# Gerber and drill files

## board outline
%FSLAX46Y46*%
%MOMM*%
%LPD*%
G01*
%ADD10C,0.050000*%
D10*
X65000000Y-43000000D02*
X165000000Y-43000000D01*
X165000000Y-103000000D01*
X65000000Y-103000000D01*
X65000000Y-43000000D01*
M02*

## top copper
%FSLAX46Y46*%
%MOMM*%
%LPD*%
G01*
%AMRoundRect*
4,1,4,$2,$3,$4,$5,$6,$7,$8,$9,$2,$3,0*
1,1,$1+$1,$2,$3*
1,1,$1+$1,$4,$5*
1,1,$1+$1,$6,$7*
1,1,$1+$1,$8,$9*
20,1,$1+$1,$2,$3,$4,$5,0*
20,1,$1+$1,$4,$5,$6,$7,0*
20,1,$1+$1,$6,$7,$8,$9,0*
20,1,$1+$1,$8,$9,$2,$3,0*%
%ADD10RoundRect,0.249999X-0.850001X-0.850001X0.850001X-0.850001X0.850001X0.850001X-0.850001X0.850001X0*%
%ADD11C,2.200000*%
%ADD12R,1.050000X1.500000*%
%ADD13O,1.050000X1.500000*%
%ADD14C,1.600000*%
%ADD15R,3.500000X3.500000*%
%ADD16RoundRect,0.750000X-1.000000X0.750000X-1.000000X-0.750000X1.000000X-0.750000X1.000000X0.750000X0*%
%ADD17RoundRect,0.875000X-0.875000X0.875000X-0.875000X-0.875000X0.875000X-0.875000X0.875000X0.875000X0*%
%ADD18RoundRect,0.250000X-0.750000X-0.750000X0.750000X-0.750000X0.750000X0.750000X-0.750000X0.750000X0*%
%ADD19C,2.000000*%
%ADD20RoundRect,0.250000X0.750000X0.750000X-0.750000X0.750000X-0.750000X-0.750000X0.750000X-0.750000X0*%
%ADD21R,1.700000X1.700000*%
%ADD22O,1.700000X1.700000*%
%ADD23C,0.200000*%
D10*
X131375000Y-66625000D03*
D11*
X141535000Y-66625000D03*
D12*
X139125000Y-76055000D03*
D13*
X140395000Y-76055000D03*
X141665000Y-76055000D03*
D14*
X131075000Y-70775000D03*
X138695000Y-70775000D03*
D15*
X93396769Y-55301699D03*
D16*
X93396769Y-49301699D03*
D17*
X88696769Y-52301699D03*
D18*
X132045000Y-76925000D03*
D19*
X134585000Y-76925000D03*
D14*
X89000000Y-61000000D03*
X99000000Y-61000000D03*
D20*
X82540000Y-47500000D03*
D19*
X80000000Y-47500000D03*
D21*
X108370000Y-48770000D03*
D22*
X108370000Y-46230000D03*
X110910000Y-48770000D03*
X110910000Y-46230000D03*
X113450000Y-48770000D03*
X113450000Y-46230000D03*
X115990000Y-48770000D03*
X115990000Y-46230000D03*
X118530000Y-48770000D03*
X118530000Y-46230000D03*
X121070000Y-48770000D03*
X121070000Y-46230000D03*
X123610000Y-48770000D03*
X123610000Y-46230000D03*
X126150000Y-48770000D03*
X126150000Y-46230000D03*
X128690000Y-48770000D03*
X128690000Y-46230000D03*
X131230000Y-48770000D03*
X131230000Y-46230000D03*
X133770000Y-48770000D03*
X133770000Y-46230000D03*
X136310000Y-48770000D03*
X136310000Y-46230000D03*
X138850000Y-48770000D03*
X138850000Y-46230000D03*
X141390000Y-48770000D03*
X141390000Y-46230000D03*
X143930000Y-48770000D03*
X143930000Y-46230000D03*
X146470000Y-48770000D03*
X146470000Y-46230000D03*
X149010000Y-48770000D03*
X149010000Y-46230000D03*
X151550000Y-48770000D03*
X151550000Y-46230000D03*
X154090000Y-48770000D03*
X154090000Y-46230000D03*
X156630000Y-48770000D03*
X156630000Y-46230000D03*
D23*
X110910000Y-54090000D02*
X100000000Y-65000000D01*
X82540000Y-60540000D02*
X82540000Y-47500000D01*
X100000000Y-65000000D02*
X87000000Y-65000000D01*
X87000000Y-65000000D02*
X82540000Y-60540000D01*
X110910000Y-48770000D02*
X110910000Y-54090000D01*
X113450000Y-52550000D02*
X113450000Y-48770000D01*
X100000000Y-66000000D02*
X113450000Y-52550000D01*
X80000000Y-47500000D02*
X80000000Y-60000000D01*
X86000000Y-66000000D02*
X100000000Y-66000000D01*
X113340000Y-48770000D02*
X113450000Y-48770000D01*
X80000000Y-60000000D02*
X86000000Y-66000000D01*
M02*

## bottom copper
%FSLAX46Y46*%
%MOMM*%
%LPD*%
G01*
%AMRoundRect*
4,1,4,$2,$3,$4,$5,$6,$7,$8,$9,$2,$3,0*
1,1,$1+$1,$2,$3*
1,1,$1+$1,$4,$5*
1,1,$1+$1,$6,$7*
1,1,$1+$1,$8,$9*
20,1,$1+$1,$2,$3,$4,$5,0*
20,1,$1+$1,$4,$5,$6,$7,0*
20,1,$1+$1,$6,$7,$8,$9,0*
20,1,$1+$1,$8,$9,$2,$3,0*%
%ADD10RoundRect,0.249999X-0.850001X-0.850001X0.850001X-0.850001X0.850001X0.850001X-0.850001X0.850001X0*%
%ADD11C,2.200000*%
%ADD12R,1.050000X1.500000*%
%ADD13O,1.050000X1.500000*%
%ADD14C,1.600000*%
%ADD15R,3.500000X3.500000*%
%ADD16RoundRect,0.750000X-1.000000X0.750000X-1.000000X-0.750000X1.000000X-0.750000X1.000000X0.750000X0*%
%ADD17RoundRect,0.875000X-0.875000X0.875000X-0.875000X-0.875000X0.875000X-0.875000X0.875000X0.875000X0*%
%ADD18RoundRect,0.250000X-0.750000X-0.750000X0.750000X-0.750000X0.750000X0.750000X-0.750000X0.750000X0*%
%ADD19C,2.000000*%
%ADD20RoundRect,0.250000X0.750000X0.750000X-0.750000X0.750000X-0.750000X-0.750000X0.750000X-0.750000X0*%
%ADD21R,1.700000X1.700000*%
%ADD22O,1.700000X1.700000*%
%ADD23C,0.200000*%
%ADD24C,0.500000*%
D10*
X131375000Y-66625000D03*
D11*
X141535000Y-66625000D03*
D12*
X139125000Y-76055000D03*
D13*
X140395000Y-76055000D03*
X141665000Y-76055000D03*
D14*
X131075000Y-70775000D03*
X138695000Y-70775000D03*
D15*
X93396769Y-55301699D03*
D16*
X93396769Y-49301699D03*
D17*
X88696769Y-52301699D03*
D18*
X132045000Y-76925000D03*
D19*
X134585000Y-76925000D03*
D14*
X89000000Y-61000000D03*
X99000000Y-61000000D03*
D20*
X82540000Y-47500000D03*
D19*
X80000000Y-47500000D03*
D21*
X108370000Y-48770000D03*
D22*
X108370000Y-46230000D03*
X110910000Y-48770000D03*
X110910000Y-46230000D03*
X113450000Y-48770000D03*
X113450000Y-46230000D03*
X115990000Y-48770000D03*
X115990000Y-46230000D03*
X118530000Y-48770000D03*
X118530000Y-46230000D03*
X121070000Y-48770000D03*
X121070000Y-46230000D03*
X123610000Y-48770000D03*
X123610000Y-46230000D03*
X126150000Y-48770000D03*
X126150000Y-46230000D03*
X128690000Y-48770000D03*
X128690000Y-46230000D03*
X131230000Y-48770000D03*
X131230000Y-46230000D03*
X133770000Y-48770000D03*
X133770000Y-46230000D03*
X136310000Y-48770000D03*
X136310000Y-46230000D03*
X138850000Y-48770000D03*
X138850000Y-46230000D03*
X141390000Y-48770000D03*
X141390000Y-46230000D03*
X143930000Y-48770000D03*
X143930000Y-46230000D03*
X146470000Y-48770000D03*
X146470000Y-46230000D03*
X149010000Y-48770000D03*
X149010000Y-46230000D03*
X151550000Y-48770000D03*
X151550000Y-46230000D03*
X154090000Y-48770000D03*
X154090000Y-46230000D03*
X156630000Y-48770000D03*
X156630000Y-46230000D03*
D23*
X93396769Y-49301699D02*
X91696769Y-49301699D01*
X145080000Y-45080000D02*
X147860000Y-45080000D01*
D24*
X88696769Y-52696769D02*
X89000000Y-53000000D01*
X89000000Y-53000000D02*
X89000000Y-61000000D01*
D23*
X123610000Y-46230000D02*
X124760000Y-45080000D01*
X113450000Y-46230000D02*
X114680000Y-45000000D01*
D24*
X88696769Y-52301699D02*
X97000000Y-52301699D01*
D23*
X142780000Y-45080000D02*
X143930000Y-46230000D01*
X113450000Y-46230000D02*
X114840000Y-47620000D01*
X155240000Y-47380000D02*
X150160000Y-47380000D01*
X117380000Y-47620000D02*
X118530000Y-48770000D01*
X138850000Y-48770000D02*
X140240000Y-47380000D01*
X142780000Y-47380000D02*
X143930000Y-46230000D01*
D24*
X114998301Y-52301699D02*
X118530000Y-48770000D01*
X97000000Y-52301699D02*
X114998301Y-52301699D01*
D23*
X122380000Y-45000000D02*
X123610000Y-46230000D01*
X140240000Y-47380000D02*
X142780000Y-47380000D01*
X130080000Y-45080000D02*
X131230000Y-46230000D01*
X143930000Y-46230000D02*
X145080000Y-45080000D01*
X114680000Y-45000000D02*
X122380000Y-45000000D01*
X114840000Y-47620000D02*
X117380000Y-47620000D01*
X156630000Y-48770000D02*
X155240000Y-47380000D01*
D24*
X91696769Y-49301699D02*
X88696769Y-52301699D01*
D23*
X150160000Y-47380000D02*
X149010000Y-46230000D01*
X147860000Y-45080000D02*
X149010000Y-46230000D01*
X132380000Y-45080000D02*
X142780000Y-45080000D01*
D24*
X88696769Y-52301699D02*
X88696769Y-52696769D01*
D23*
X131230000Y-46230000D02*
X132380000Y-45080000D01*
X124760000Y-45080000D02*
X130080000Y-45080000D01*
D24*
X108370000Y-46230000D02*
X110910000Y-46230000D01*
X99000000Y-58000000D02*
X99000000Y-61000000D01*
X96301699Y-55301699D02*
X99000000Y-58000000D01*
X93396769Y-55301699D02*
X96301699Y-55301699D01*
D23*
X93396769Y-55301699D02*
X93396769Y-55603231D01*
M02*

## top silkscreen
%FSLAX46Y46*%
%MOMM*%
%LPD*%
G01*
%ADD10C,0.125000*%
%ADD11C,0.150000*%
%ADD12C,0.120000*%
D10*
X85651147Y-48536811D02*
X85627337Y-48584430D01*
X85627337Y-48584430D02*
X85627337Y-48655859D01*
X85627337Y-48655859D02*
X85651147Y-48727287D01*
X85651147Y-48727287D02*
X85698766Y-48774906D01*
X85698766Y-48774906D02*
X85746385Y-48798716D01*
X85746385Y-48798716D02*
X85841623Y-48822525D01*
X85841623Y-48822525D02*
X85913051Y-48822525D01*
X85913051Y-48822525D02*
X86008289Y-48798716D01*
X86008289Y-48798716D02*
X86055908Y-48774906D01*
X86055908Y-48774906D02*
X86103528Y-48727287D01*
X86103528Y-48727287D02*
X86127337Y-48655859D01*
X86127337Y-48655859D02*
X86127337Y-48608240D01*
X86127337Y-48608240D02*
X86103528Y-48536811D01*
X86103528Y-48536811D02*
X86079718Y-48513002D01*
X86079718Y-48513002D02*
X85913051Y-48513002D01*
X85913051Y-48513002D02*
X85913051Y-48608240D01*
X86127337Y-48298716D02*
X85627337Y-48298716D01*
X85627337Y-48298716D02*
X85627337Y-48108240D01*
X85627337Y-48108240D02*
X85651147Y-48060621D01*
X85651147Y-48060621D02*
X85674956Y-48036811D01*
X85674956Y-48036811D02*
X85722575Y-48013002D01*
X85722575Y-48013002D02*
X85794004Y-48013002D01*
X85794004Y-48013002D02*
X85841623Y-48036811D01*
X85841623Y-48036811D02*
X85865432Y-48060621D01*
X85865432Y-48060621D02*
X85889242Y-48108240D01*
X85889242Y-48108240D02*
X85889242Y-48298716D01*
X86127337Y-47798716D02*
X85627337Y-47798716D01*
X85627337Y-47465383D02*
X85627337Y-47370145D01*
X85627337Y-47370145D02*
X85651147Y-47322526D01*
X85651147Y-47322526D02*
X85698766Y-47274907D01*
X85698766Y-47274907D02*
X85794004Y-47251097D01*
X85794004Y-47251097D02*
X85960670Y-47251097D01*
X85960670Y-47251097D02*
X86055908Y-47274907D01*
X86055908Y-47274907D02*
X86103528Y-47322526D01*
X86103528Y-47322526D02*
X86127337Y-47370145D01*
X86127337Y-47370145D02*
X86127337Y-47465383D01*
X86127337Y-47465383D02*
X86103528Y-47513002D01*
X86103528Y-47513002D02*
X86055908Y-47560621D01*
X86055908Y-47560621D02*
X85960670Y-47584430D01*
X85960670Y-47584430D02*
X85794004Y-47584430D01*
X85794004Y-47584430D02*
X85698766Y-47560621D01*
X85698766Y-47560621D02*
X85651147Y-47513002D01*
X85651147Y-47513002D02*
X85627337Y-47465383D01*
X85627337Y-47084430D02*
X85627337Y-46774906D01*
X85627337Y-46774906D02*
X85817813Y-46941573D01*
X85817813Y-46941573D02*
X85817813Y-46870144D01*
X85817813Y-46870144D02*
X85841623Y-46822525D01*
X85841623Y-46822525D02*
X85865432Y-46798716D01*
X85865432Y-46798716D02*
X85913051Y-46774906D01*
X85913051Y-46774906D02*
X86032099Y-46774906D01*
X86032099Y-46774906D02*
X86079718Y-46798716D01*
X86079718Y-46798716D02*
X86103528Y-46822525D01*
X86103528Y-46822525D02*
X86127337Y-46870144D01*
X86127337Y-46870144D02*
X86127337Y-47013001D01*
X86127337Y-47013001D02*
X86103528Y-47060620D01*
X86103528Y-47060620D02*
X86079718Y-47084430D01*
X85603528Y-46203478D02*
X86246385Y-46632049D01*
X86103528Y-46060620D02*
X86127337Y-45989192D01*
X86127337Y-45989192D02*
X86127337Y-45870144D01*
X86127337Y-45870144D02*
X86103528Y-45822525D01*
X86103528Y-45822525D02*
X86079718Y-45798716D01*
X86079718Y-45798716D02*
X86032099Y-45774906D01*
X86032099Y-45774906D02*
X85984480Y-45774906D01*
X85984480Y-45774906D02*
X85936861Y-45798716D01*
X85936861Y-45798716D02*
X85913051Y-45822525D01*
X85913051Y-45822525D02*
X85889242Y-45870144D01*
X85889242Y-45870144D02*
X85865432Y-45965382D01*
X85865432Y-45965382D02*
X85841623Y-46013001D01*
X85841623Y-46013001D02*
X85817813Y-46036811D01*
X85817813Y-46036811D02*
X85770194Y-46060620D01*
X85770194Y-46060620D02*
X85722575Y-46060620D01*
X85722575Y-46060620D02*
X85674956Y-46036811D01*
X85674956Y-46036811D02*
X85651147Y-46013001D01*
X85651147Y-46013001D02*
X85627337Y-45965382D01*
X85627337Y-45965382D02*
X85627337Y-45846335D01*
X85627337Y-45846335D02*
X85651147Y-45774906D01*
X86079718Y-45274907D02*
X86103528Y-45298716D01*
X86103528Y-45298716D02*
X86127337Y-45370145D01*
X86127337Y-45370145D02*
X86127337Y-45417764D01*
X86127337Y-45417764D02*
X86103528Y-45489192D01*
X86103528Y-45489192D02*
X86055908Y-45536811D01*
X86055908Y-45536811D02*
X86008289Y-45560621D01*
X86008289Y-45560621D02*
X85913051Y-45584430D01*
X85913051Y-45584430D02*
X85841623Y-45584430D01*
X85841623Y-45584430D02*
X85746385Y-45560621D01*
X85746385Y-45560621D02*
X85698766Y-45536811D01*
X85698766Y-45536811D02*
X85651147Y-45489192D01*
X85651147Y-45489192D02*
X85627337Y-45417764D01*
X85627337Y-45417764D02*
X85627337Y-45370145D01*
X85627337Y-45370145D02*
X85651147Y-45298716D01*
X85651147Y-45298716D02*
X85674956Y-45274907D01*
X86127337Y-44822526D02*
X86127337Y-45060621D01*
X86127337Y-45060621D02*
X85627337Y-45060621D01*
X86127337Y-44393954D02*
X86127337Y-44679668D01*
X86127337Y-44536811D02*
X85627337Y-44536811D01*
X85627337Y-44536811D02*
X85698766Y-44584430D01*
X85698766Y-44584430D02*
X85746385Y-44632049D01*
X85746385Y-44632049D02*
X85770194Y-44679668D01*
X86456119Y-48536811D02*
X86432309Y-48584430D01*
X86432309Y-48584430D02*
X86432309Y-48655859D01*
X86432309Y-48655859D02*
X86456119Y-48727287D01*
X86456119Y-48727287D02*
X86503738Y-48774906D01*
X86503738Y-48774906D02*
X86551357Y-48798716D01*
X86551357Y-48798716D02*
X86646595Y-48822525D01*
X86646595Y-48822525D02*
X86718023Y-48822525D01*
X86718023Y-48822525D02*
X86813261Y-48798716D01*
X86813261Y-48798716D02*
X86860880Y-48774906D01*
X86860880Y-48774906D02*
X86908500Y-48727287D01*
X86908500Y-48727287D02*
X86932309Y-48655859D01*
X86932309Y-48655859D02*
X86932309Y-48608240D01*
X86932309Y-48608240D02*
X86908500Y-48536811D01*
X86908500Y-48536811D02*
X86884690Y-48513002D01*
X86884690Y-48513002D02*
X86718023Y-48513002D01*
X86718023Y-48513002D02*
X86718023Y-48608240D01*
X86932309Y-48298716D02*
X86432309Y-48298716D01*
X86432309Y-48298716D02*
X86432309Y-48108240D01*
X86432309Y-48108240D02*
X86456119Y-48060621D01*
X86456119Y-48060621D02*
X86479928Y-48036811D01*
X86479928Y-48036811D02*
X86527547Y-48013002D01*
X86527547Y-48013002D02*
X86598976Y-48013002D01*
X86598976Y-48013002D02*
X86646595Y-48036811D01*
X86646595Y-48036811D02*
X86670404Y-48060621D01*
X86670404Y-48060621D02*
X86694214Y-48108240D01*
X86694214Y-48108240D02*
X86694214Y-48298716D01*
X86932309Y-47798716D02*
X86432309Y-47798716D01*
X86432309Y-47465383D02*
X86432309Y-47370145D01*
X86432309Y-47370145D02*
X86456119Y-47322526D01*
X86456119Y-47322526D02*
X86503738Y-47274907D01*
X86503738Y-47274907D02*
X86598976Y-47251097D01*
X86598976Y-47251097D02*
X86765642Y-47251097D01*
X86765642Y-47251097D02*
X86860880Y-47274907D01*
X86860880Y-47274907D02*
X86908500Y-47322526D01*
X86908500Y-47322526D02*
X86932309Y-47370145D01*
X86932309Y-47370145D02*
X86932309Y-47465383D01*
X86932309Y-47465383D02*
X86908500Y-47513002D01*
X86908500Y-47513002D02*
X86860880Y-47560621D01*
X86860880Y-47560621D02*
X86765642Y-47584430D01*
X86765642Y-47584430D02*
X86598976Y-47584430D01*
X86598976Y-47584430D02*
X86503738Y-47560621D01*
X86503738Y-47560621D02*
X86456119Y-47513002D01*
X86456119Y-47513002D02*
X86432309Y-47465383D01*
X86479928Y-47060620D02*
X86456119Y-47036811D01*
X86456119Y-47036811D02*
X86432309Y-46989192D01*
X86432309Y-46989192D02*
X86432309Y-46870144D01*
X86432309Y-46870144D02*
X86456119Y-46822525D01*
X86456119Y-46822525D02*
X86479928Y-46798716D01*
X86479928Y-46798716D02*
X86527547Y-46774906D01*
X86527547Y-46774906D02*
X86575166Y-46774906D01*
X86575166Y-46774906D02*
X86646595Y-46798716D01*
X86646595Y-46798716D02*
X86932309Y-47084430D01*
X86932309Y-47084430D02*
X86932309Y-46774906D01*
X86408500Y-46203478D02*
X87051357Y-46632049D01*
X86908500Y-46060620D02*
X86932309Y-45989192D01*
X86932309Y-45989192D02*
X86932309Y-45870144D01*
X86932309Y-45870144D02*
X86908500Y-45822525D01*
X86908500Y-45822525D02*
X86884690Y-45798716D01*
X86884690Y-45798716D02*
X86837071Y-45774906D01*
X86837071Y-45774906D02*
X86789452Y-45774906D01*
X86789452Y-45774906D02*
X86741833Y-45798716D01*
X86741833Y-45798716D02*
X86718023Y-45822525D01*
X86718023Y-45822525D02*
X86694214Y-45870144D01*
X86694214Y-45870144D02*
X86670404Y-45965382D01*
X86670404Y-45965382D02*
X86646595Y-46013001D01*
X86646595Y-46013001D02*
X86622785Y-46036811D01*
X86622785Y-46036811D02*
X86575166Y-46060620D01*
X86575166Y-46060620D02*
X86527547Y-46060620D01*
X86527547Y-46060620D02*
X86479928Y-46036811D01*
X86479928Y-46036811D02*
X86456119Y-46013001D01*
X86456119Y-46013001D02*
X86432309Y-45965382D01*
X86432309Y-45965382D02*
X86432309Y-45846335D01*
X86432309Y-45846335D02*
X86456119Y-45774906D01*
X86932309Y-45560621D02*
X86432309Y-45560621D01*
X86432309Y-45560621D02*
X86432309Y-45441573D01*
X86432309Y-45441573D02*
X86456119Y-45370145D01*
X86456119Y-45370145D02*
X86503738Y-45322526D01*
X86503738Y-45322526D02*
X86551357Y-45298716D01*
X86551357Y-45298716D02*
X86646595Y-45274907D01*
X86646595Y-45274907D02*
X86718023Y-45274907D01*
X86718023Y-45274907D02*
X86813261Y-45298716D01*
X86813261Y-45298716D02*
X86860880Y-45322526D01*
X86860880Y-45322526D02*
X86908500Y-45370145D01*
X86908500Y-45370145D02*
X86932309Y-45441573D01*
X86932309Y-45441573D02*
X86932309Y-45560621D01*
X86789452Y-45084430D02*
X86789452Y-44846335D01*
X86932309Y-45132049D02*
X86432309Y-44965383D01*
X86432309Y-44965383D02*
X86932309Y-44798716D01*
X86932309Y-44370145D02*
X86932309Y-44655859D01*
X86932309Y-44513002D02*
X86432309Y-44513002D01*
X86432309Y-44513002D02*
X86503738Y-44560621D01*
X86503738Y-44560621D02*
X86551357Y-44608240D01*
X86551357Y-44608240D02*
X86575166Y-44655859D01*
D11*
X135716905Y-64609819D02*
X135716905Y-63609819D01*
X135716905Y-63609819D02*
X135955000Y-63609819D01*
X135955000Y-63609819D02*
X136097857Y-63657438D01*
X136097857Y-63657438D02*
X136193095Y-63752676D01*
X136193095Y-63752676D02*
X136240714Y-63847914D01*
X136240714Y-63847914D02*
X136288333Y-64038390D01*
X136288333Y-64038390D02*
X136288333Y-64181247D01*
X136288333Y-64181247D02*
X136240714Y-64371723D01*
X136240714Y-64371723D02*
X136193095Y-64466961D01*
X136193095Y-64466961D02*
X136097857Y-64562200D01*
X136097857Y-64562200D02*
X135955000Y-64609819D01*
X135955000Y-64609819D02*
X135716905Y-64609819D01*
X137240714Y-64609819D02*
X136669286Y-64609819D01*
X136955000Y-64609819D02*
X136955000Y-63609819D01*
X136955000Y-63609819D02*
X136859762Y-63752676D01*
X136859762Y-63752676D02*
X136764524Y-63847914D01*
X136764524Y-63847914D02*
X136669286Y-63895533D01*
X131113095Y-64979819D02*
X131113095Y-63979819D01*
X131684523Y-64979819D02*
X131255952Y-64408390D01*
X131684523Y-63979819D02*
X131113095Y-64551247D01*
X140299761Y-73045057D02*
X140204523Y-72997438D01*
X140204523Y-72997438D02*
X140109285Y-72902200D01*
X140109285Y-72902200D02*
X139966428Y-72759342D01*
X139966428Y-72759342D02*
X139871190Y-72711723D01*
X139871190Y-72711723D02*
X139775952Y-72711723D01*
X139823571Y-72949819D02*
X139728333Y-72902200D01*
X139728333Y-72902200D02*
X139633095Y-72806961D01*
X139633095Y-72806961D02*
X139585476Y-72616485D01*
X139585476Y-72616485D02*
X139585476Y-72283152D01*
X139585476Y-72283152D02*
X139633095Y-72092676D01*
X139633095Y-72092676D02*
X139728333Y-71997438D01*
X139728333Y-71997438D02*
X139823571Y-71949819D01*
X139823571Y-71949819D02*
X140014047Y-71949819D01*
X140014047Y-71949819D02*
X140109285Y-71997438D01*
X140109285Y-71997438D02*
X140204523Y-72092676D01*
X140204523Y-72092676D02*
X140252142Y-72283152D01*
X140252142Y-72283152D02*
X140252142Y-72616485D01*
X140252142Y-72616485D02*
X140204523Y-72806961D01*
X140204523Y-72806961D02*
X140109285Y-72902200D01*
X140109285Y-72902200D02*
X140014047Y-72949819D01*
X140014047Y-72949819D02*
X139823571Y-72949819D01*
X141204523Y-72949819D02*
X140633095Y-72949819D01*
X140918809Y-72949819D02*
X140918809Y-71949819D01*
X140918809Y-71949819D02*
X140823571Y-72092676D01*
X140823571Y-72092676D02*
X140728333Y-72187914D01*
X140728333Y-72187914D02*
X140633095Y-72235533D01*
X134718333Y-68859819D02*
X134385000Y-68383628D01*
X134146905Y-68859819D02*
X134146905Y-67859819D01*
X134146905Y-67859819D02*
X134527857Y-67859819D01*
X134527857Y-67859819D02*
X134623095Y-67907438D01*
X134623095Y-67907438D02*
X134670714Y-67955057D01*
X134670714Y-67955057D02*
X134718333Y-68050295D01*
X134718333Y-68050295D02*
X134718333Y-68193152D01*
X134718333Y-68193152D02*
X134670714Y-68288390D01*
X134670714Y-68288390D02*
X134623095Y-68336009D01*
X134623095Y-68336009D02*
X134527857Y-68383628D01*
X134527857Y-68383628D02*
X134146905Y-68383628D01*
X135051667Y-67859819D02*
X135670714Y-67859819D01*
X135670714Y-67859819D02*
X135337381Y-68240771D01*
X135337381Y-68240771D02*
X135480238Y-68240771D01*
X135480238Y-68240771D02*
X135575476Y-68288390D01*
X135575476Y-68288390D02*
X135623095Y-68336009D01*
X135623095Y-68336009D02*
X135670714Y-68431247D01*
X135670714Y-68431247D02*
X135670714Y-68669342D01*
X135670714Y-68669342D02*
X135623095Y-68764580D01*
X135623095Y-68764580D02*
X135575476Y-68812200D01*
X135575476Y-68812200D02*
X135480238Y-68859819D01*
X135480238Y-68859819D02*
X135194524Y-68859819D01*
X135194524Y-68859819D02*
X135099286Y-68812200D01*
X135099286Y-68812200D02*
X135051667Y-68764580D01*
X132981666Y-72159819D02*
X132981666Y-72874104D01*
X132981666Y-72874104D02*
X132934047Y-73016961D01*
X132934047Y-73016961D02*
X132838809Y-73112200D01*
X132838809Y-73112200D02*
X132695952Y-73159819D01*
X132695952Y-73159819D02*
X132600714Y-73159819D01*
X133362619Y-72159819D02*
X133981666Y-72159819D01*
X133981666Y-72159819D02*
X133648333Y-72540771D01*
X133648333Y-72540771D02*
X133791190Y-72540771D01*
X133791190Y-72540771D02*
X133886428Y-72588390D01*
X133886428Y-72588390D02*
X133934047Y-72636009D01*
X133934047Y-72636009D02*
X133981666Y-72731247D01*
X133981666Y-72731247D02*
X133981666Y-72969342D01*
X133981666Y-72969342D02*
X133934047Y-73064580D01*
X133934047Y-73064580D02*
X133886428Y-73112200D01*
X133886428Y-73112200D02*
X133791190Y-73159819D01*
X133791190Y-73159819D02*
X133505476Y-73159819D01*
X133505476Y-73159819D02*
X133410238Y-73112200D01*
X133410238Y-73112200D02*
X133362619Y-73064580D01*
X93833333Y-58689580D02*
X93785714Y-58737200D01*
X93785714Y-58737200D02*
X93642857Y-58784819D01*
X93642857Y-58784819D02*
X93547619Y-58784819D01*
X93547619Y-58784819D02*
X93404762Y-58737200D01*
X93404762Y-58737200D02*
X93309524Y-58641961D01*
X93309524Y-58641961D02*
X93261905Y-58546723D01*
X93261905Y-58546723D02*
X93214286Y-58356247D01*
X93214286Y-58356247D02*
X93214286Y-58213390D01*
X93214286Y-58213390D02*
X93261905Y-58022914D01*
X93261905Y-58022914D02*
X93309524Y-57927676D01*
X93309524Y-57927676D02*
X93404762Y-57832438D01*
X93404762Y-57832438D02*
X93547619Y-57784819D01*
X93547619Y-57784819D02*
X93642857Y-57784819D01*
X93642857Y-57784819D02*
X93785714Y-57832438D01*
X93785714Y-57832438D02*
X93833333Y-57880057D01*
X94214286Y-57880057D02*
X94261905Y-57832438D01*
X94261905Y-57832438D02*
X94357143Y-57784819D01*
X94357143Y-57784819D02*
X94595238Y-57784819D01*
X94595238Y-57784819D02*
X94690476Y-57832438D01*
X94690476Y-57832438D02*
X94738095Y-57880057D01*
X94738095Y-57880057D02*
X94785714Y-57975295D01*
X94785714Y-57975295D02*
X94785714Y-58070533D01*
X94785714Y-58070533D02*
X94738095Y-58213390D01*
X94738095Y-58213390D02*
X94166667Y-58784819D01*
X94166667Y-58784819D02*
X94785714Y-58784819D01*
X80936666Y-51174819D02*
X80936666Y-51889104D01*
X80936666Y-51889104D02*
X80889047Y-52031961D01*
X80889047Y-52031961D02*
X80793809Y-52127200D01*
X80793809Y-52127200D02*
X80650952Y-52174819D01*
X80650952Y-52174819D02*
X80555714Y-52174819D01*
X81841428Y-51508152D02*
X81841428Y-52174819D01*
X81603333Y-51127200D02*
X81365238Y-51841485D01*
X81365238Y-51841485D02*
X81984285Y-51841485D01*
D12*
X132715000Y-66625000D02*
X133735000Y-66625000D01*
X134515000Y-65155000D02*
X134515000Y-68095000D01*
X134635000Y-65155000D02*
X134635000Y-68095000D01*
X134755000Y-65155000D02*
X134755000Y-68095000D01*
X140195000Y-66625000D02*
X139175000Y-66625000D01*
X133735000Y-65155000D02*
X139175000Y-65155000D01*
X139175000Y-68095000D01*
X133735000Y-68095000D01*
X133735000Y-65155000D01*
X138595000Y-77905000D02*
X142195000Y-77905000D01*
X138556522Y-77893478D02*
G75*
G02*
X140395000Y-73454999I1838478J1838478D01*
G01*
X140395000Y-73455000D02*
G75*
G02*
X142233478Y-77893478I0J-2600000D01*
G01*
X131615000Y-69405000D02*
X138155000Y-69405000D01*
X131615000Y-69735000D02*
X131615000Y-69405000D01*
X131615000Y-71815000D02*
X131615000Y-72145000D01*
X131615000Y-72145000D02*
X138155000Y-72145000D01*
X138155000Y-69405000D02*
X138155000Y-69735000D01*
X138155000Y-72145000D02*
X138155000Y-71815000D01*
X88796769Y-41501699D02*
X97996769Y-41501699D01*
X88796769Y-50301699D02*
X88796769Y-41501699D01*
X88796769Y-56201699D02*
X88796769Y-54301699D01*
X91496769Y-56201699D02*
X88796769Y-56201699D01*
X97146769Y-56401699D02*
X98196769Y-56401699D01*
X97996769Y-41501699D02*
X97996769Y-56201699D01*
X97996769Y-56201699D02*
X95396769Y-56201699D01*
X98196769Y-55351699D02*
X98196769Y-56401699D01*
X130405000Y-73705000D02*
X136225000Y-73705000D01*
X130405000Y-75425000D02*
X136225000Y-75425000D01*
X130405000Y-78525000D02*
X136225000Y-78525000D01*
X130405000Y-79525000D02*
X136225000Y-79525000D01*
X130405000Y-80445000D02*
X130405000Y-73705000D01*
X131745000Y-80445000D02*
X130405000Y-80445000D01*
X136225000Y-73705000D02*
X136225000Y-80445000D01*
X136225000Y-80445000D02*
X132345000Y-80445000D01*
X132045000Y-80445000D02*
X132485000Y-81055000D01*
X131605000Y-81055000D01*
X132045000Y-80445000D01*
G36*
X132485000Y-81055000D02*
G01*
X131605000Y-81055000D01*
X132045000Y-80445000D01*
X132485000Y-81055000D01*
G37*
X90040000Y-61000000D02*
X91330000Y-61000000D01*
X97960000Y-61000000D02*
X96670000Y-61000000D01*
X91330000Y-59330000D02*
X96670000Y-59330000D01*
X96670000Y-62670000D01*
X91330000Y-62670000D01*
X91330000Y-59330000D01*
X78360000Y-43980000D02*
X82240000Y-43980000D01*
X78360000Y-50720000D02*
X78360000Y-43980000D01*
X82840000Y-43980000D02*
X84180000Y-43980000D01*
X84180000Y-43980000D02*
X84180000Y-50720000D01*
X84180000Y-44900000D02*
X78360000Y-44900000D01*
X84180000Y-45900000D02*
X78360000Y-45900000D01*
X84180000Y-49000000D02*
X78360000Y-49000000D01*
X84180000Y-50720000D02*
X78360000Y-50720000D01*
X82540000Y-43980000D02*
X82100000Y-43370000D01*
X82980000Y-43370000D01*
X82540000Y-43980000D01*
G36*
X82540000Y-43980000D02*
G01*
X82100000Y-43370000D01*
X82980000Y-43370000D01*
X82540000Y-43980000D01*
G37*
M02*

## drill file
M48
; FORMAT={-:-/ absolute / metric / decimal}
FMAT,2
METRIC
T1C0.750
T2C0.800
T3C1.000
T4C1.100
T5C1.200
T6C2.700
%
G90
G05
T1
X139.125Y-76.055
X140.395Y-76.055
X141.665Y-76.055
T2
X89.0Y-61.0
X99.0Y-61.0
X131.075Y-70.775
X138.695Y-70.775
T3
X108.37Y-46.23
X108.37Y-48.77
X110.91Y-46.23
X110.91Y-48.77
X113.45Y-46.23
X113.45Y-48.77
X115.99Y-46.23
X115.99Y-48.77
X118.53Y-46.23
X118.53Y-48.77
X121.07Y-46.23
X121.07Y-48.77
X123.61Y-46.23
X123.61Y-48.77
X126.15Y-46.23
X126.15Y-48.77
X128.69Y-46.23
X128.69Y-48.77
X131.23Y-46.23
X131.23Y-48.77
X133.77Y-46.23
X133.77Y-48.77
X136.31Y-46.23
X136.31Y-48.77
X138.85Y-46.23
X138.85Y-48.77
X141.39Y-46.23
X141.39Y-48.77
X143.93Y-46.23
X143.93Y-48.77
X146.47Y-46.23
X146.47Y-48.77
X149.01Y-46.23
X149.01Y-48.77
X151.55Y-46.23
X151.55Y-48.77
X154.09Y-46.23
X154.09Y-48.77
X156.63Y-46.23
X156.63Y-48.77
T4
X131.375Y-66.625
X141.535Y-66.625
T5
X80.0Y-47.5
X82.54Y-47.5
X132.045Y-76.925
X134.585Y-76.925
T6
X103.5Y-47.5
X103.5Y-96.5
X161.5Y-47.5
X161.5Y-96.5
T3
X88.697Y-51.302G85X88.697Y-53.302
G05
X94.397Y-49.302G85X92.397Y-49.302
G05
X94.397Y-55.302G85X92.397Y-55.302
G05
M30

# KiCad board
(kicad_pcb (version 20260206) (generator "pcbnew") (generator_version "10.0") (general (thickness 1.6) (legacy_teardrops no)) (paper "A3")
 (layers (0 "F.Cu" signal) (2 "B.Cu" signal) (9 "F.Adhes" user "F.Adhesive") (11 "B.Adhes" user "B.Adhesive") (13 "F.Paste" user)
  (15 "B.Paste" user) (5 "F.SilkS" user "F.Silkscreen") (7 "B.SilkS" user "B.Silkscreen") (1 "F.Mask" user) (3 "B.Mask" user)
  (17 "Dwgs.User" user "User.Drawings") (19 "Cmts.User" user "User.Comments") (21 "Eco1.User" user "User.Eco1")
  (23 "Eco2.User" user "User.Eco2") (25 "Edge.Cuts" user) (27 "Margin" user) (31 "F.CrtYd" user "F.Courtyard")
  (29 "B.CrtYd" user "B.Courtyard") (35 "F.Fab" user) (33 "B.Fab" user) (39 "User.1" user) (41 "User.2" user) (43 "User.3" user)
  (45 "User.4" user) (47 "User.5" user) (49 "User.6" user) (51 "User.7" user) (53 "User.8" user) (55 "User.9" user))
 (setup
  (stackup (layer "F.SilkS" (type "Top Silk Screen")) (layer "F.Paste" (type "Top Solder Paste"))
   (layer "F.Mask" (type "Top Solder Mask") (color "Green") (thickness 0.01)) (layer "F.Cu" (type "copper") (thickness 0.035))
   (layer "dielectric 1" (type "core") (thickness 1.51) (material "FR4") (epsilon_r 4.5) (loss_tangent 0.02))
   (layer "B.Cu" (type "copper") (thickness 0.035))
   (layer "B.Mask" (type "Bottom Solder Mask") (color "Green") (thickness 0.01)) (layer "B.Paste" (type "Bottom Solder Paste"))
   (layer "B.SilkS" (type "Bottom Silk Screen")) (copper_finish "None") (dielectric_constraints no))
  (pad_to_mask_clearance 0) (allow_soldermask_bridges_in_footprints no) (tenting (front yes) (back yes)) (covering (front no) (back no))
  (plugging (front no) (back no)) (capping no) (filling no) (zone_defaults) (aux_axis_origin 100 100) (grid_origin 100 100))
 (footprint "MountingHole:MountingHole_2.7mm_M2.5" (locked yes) (layer "F.Cu") (at 161.5 47.5)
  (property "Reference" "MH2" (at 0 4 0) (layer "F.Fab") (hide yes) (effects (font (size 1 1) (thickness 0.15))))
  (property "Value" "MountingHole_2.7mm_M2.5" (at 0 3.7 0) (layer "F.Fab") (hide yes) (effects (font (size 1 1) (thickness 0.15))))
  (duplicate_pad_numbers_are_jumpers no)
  (pad "" np_thru_hole circle (at 0 0) (size 2.7 2.7) (drill 2.7) (layers "*.Cu" "*.Mask")))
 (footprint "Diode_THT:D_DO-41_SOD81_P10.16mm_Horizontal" (layer "F.Cu") (at 131.375 66.625)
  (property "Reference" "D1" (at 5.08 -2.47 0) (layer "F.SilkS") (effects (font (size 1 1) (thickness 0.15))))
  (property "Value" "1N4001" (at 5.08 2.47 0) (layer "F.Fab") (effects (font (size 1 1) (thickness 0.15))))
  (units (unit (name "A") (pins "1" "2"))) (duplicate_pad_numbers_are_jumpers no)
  (fp_line (start 1.34 0) (end 2.36 0) (stroke (width 0.12) (type solid)) (layer "F.SilkS"))
  (fp_line (start 3.14 -1.47) (end 3.14 1.47) (stroke (width 0.12) (type solid)) (layer "F.SilkS"))
  (fp_line (start 3.26 -1.47) (end 3.26 1.47) (stroke (width 0.12) (type solid)) (layer "F.SilkS"))
  (fp_line (start 3.38 -1.47) (end 3.38 1.47) (stroke (width 0.12) (type solid)) (layer "F.SilkS"))
  (fp_line (start 8.82 0) (end 7.8 0) (stroke (width 0.12) (type solid)) (layer "F.SilkS"))
  (fp_rect (start 2.36 -1.47) (end 7.8 1.47) (stroke (width 0.12) (type solid)) (fill no) (layer "F.SilkS"))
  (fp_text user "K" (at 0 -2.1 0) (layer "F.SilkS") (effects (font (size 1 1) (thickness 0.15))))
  (pad "1" thru_hole roundrect (at 0 0) (size 2.2 2.2) (drill 1.1) (layers "*.Cu" "*.Mask") (remove_unused_layers no)
   (roundrect_rratio 0.113636) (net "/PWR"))
  (pad "2" thru_hole circle (at 10.16 0) (size 2.2 2.2) (drill 1.1) (layers "*.Cu" "*.Mask") (remove_unused_layers no) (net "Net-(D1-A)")))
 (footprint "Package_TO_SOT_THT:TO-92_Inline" (layer "F.Cu") (at 139.125 76.055)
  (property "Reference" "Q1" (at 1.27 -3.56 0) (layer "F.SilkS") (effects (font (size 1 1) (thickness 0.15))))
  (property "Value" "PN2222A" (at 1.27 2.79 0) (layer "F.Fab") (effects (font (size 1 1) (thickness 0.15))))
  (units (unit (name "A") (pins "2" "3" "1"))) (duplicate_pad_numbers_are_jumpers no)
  (fp_line (start -0.53 1.85) (end 3.07 1.85) (stroke (width 0.12) (type solid)) (layer "F.SilkS"))
  (fp_arc (start -0.568478 1.838478) (mid -1.132087 -0.994977) (end 1.27 -2.6) (stroke (width 0.12) (type solid)) (layer "F.SilkS"))
  (fp_arc (start 1.27 -2.6) (mid 3.672087 -0.994977) (end 3.108478 1.838478) (stroke (width 0.12) (type solid)) (layer "F.SilkS"))
  (pad "1" thru_hole rect (at 0 0) (size 1.05 1.5) (drill 0.75) (layers "*.Cu" "*.Mask") (remove_unused_layers no) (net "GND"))
  (pad "2" thru_hole oval (at 1.27 0) (size 1.05 1.5) (drill 0.75) (layers "*.Cu" "*.Mask") (remove_unused_layers no) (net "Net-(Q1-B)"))
  (pad "3" thru_hole oval (at 2.54 0) (size 1.05 1.5) (drill 0.75) (layers "*.Cu" "*.Mask") (remove_unused_layers no) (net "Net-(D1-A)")))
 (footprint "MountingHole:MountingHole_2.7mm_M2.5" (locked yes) (layer "F.Cu") (at 103.5 96.5)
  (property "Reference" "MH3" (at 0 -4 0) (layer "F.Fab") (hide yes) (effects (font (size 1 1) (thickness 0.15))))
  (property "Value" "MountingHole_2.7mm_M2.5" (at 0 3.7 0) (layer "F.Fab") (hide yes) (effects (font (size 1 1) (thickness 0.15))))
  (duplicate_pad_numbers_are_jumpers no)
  (pad "" np_thru_hole circle (at 0 0) (size 2.7 2.7) (drill 2.7) (layers "*.Cu" "*.Mask")))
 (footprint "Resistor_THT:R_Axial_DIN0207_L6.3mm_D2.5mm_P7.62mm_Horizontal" (layer "F.Cu") (at 131.075 70.775)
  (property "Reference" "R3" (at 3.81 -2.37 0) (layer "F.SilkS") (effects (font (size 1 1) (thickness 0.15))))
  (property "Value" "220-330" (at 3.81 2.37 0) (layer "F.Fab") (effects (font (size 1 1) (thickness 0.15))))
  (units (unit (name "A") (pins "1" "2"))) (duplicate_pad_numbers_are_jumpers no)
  (fp_line (start 0.54 -1.37) (end 7.08 -1.37) (stroke (width 0.12) (type solid)) (layer "F.SilkS"))
  (fp_line (start 0.54 -1.04) (end 0.54 -1.37) (stroke (width 0.12) (type solid)) (layer "F.SilkS"))
  (fp_line (start 0.54 1.04) (end 0.54 1.37) (stroke (width 0.12) (type solid)) (layer "F.SilkS"))
  (fp_line (start 0.54 1.37) (end 7.08 1.37) (stroke (width 0.12) (type solid)) (layer "F.SilkS"))
  (fp_line (start 7.08 -1.37) (end 7.08 -1.04) (stroke (width 0.12) (type solid)) (layer "F.SilkS"))
  (fp_line (start 7.08 1.37) (end 7.08 1.04) (stroke (width 0.12) (type solid)) (layer "F.SilkS"))
  (pad "1" thru_hole circle (at 0 0) (size 1.6 1.6) (drill 0.8) (layers "*.Cu" "*.Mask") (remove_unused_layers no) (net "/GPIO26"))
  (pad "2" thru_hole circle (at 7.62 0) (size 1.6 1.6) (drill 0.8) (layers "*.Cu" "*.Mask") (remove_unused_layers no) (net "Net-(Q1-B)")))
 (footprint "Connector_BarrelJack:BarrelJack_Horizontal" (layer "F.Cu") (at 93.396769 55.301699 -90)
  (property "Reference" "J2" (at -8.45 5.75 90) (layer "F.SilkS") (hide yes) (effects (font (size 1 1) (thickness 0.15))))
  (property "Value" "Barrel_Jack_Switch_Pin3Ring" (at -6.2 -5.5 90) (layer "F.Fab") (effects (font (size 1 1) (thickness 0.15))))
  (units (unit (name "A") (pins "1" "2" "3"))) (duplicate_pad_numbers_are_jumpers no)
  (fp_line (start -13.8 4.6) (end -13.8 -4.6) (stroke (width 0.12) (type solid)) (layer "F.SilkS"))
  (fp_line (start -5 4.6) (end -13.8 4.6) (stroke (width 0.12) (type solid)) (layer "F.SilkS"))
  (fp_line (start 0.9 4.6) (end -1 4.6) (stroke (width 0.12) (type solid)) (layer "F.SilkS"))
  (fp_line (start 0.9 1.9) (end 0.9 4.6) (stroke (width 0.12) (type solid)) (layer "F.SilkS"))
  (fp_line (start 1.1 -3.75) (end 1.1 -4.8) (stroke (width 0.12) (type solid)) (layer "F.SilkS"))
  (fp_line (start -13.8 -4.6) (end 0.9 -4.6) (stroke (width 0.12) (type solid)) (layer "F.SilkS"))
  (fp_line (start 0.9 -4.6) (end 0.9 -2) (stroke (width 0.12) (type solid)) (layer "F.SilkS"))
  (fp_line (start 0.05 -4.8) (end 1.1 -4.8) (stroke (width 0.12) (type solid)) (layer "F.SilkS"))
  (pad "1" thru_hole rect (at 0 0 270) (size 3.5 3.5) (drill oval 1 3) (layers "*.Cu" "*.Mask") (remove_unused_layers no) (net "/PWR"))
  (pad "2" thru_hole roundrect (at -6 0 270) (size 3 3.5) (drill oval 1 3) (layers "*.Cu" "*.Mask") (remove_unused_layers no)
   (roundrect_rratio 0.25) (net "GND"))
  (pad "3" thru_hole roundrect (at -3 4.7 270) (size 3.5 3.5) (drill oval 3 1) (layers "*.Cu" "*.Mask") (remove_unused_layers no)
   (roundrect_rratio 0.25) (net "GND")))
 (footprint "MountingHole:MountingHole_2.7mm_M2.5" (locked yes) (layer "F.Cu") (at 103.5 47.5)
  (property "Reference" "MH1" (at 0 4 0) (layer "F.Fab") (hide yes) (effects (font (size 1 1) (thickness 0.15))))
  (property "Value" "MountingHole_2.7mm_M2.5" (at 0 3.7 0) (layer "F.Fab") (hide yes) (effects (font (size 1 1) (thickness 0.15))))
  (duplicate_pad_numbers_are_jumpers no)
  (pad "" np_thru_hole circle (at 0 0) (size 2.7 2.7) (drill 2.7) (layers "*.Cu" "*.Mask")))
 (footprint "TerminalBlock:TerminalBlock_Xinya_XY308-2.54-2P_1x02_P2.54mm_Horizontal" (layer "F.Cu") (at 132.045 76.925)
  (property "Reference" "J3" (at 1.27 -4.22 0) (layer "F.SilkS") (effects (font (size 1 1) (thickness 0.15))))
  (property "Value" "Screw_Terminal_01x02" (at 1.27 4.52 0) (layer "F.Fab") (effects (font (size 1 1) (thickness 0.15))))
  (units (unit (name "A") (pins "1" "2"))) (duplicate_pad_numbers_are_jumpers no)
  (fp_line (start -1.64 -3.22) (end 4.18 -3.22) (stroke (width 0.12) (type solid)) (layer "F.SilkS"))
  (fp_line (start -1.64 -1.5) (end 4.18 -1.5) (stroke (width 0.12) (type solid)) (layer "F.SilkS"))
  (fp_line (start -1.64 1.6) (end 4.18 1.6) (stroke (width 0.12) (type solid)) (layer "F.SilkS"))
  (fp_line (start -1.64 2.6) (end 4.18 2.6) (stroke (width 0.12) (type solid)) (layer "F.SilkS"))
  (fp_line (start -1.64 3.52) (end -1.64 -3.22) (stroke (width 0.12) (type solid)) (layer "F.SilkS"))
  (fp_line (start -0.3 3.52) (end -1.64 3.52) (stroke (width 0.12) (type solid)) (layer "F.SilkS"))
  (fp_line (start 4.18 -3.22) (end 4.18 3.52) (stroke (width 0.12) (type solid)) (layer "F.SilkS"))
  (fp_line (start 4.18 3.52) (end 0.3 3.52) (stroke (width 0.12) (type solid)) (layer "F.SilkS"))
  (fp_poly (pts (xy 0 3.52) (xy 0.44 4.13) (xy -0.44 4.13)) (stroke (width 0.12) (type solid)) (fill yes) (layer "F.SilkS"))
  (pad "1" thru_hole roundrect (at 0 0) (size 2 2) (drill 1.2) (layers "*.Cu" "*.Mask") (remove_unused_layers no) (roundrect_rratio 0.125)
   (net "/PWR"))
  (pad "2" thru_hole circle (at 2.54 0) (size 2 2) (drill 1.2) (layers "*.Cu" "*.Mask") (remove_unused_layers no) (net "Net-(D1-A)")))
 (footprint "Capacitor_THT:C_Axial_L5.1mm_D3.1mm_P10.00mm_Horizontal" (layer "F.Cu") (at 89 61)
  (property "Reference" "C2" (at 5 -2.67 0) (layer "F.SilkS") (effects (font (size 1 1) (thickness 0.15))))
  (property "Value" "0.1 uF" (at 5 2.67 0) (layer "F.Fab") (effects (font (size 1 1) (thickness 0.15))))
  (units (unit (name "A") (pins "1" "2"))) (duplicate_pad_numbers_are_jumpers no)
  (fp_line (start 1.04 0) (end 2.33 0) (stroke (width 0.12) (type solid)) (layer "F.SilkS"))
  (fp_line (start 8.96 0) (end 7.67 0) (stroke (width 0.12) (type solid)) (layer "F.SilkS"))
  (fp_rect (start 2.33 -1.67) (end 7.67 1.67) (stroke (width 0.12) (type solid)) (fill no) (layer "F.SilkS"))
  (pad "1" thru_hole circle (at 0 0) (size 1.6 1.6) (drill 0.8) (layers "*.Cu" "*.Mask") (remove_unused_layers no) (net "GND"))
  (pad "2" thru_hole circle (at 10 0) (size 1.6 1.6) (drill 0.8) (layers "*.Cu" "*.Mask") (remove_unused_layers no) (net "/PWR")))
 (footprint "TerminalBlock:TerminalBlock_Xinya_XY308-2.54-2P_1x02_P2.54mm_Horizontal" (layer "F.Cu") (at 82.54 47.5 180)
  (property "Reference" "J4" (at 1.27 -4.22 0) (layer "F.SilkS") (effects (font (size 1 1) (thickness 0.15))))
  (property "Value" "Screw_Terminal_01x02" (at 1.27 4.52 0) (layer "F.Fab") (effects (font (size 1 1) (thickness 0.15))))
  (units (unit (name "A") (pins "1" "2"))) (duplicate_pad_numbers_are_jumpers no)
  (fp_line (start 4.18 3.52) (end 0.3 3.52) (stroke (width 0.12) (type solid)) (layer "F.SilkS"))
  (fp_line (start 4.18 -3.22) (end 4.18 3.52) (stroke (width 0.12) (type solid)) (layer "F.SilkS"))
  (fp_line (start -0.3 3.52) (end -1.64 3.52) (stroke (width 0.12) (type solid)) (layer "F.SilkS"))
  (fp_line (start -1.64 3.52) (end -1.64 -3.22) (stroke (width 0.12) (type solid)) (layer "F.SilkS"))
  (fp_line (start -1.64 2.6) (end 4.18 2.6) (stroke (width 0.12) (type solid)) (layer "F.SilkS"))
  (fp_line (start -1.64 1.6) (end 4.18 1.6) (stroke (width 0.12) (type solid)) (layer "F.SilkS"))
  (fp_line (start -1.64 -1.5) (end 4.18 -1.5) (stroke (width 0.12) (type solid)) (layer "F.SilkS"))
  (fp_line (start -1.64 -3.22) (end 4.18 -3.22) (stroke (width 0.12) (type solid)) (layer "F.SilkS"))
  (fp_poly (pts (xy 0 3.52) (xy 0.44 4.13) (xy -0.44 4.13)) (stroke (width 0.12) (type solid)) (fill yes) (layer "F.SilkS"))
  (pad "1" thru_hole roundrect (at 0 0 180) (size 2 2) (drill 1.2) (layers "*.Cu" "*.Mask") (remove_unused_layers no)
   (roundrect_rratio 0.125) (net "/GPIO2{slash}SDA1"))
  (pad "2" thru_hole circle (at 2.54 0 180) (size 2 2) (drill 1.2) (layers "*.Cu" "*.Mask") (remove_unused_layers no)
   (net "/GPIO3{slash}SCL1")))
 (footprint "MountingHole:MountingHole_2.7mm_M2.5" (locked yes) (layer "F.Cu") (at 161.5 96.5)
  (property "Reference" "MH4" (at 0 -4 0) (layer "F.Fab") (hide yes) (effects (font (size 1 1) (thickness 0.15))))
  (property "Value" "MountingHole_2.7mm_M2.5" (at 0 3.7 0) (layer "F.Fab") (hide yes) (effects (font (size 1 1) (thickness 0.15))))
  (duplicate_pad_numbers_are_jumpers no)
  (pad "" np_thru_hole circle (at 0 0) (size 2.7 2.7) (drill 2.7) (layers "*.Cu" "*.Mask")))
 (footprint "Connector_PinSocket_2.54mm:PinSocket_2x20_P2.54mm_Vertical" (layer "B.Cu") (at 108.37 48.77 -90)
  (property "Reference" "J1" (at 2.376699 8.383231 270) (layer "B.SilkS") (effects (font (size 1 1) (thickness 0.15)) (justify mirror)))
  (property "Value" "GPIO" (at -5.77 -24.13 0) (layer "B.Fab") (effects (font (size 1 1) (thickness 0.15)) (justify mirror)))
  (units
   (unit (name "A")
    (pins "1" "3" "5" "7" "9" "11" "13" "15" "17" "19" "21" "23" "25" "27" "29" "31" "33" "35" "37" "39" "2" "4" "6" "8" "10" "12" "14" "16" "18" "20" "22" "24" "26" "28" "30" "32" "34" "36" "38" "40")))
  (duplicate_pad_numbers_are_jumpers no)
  (pad "1" thru_hole rect (at 0 0 270) (size 1.7 1.7) (drill 1) (layers "*.Cu" "*.Mask") (remove_unused_layers no) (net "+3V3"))
  (pad "2" thru_hole oval (at -2.54 0 270) (size 1.7 1.7) (drill 1) (layers "*.Cu" "*.Mask") (remove_unused_layers no) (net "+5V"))
  (pad "3" thru_hole oval (at 0 -2.54 270) (size 1.7 1.7) (drill 1) (layers "*.Cu" "*.Mask") (remove_unused_layers no)
   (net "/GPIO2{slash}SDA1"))
  (pad "4" thru_hole oval (at -2.54 -2.54 270) (size 1.7 1.7) (drill 1) (layers "*.Cu" "*.Mask") (remove_unused_layers no) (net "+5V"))
  (pad "5" thru_hole oval (at 0 -5.08 270) (size 1.7 1.7) (drill 1) (layers "*.Cu" "*.Mask") (remove_unused_layers no)
   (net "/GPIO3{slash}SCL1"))
  (pad "6" thru_hole oval (at -2.54 -5.08 270) (size 1.7 1.7) (drill 1) (layers "*.Cu" "*.Mask") (remove_unused_layers no) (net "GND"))
  (pad "7" thru_hole oval (at 0 -7.62 270) (size 1.7 1.7) (drill 1) (layers "*.Cu" "*.Mask") (remove_unused_layers no)
   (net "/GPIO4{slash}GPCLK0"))
  (pad "8" thru_hole oval (at -2.54 -7.62 270) (size 1.7 1.7) (drill 1) (layers "*.Cu" "*.Mask") (remove_unused_layers no)
   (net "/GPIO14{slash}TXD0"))
  (pad "9" thru_hole oval (at 0 -10.16 270) (size 1.7 1.7) (drill 1) (layers "*.Cu" "*.Mask") (remove_unused_layers no) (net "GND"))
  (pad "10" thru_hole oval (at -2.54 -10.16 270) (size 1.7 1.7) (drill 1) (layers "*.Cu" "*.Mask") (remove_unused_layers no)
   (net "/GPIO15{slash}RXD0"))
  (pad "11" thru_hole oval (at 0 -12.7 270) (size 1.7 1.7) (drill 1) (layers "*.Cu" "*.Mask") (remove_unused_layers no) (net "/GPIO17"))
  (pad "12" thru_hole oval (at -2.54 -12.7 270) (size 1.7 1.7) (drill 1) (layers "*.Cu" "*.Mask") (remove_unused_layers no)
   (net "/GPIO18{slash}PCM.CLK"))
  (pad "13" thru_hole oval (at 0 -15.24 270) (size 1.7 1.7) (drill 1) (layers "*.Cu" "*.Mask") (remove_unused_layers no) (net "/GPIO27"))
  (pad "14" thru_hole oval (at -2.54 -15.24 270) (size 1.7 1.7) (drill 1) (layers "*.Cu" "*.Mask") (remove_unused_layers no) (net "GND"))
  (pad "15" thru_hole oval (at 0 -17.78 270) (size 1.7 1.7) (drill 1) (layers "*.Cu" "*.Mask") (remove_unused_layers no) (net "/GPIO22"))
  (pad "16" thru_hole oval (at -2.54 -17.78 270) (size 1.7 1.7) (drill 1) (layers "*.Cu" "*.Mask") (remove_unused_layers no) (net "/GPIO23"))
  (pad "17" thru_hole oval (at 0 -20.32 270) (size 1.7 1.7) (drill 1) (layers "*.Cu" "*.Mask") (remove_unused_layers no) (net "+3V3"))
  (pad "18" thru_hole oval (at -2.54 -20.32 270) (size 1.7 1.7) (drill 1) (layers "*.Cu" "*.Mask") (remove_unused_layers no) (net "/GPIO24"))
  (pad "19" thru_hole oval (at 0 -22.86 270) (size 1.7 1.7) (drill 1) (layers "*.Cu" "*.Mask") (remove_unused_layers no)
   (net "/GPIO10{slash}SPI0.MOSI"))
  (pad "20" thru_hole oval (at -2.54 -22.86 270) (size 1.7 1.7) (drill 1) (layers "*.Cu" "*.Mask") (remove_unused_layers no) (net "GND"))
  (pad "21" thru_hole oval (at 0 -25.4 270) (size 1.7 1.7) (drill 1) (layers "*.Cu" "*.Mask") (remove_unused_layers no)
   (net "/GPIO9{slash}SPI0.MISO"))
  (pad "22" thru_hole oval (at -2.54 -25.4 270) (size 1.7 1.7) (drill 1) (layers "*.Cu" "*.Mask") (remove_unused_layers no) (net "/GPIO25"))
  (pad "23" thru_hole oval (at 0 -27.94 270) (size 1.7 1.7) (drill 1) (layers "*.Cu" "*.Mask") (remove_unused_layers no)
   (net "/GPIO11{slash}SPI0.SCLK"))
  (pad "24" thru_hole oval (at -2.54 -27.94 270) (size 1.7 1.7) (drill 1) (layers "*.Cu" "*.Mask") (remove_unused_layers no)
   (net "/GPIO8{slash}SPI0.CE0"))
  (pad "25" thru_hole oval (at 0 -30.48 270) (size 1.7 1.7) (drill 1) (layers "*.Cu" "*.Mask") (remove_unused_layers no) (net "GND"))
  (pad "26" thru_hole oval (at -2.54 -30.48 270) (size 1.7 1.7) (drill 1) (layers "*.Cu" "*.Mask") (remove_unused_layers no)
   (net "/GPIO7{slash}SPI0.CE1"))
  (pad "27" thru_hole oval (at 0 -33.02 270) (size 1.7 1.7) (drill 1) (layers "*.Cu" "*.Mask") (remove_unused_layers no) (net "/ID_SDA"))
  (pad "28" thru_hole oval (at -2.54 -33.02 270) (size 1.7 1.7) (drill 1) (layers "*.Cu" "*.Mask") (remove_unused_layers no) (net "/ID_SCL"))
  (pad "29" thru_hole oval (at 0 -35.56 270) (size 1.7 1.7) (drill 1) (layers "*.Cu" "*.Mask") (remove_unused_layers no) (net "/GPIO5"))
  (pad "30" thru_hole oval (at -2.54 -35.56 270) (size 1.7 1.7) (drill 1) (layers "*.Cu" "*.Mask") (remove_unused_layers no) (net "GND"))
  (pad "31" thru_hole oval (at 0 -38.1 270) (size 1.7 1.7) (drill 1) (layers "*.Cu" "*.Mask") (remove_unused_layers no) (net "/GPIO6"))
  (pad "32" thru_hole oval (at -2.54 -38.1 270) (size 1.7 1.7) (drill 1) (layers "*.Cu" "*.Mask") (remove_unused_layers no)
   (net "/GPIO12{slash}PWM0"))
  (pad "33" thru_hole oval (at 0 -40.64 270) (size 1.7 1.7) (drill 1) (layers "*.Cu" "*.Mask") (remove_unused_layers no)
   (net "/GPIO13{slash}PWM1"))
  (pad "34" thru_hole oval (at -2.54 -40.64 270) (size 1.7 1.7) (drill 1) (layers "*.Cu" "*.Mask") (remove_unused_layers no) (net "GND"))
  (pad "35" thru_hole oval (at 0 -43.18 270) (size 1.7 1.7) (drill 1) (layers "*.Cu" "*.Mask") (remove_unused_layers no)
   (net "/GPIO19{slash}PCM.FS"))
  (pad "36" thru_hole oval (at -2.54 -43.18 270) (size 1.7 1.7) (drill 1) (layers "*.Cu" "*.Mask") (remove_unused_layers no) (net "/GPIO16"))
  (pad "37" thru_hole oval (at 0 -45.72 270) (size 1.7 1.7) (drill 1) (layers "*.Cu" "*.Mask") (remove_unused_layers no) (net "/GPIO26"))
  (pad "38" thru_hole oval (at -2.54 -45.72 270) (size 1.7 1.7) (drill 1) (layers "*.Cu" "*.Mask") (remove_unused_layers no)
   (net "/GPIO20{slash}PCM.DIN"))
  (pad "39" thru_hole oval (at 0 -48.26 270) (size 1.7 1.7) (drill 1) (layers "*.Cu" "*.Mask") (remove_unused_layers no) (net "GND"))
  (pad "40" thru_hole oval (at -2.54 -48.26 270) (size 1.7 1.7) (drill 1) (layers "*.Cu" "*.Mask") (remove_unused_layers no)
   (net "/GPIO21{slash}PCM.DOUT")))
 (gr_rect (start 65 43) (end 165 103) (stroke (width 0.05) (type default)) (fill no) (layer "Edge.Cuts"))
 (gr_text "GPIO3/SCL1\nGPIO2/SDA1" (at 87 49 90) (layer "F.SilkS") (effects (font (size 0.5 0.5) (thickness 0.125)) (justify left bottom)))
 (segment (start 93.396769 49.301699) (end 91.696769 49.301699) (width 0.2) (layer "B.Cu") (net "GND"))
 (segment (start 145.08 45.08) (end 147.86 45.08) (width 0.2) (layer "B.Cu") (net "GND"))
 (segment (start 88.696769 52.696769) (end 89 53) (width 0.5) (layer "B.Cu") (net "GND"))
 (segment (start 89 53) (end 89 61) (width 0.5) (layer "B.Cu") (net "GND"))
 (segment (start 123.61 46.23) (end 124.76 45.08) (width 0.2) (layer "B.Cu") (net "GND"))
 (segment (start 113.45 46.23) (end 114.68 45) (width 0.2) (layer "B.Cu") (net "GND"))
 (segment (start 88.696769 52.301699) (end 97 52.301699) (width 0.5) (layer "B.Cu") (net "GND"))
 (segment (start 142.78 45.08) (end 143.93 46.23) (width 0.2) (layer "B.Cu") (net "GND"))
 (segment (start 113.45 46.23) (end 114.84 47.62) (width 0.2) (layer "B.Cu") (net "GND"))
 (segment (start 155.24 47.38) (end 150.16 47.38) (width 0.2) (layer "B.Cu") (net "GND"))
 (segment (start 117.38 47.62) (end 118.53 48.77) (width 0.2) (layer "B.Cu") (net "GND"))
 (segment (start 138.85 48.77) (end 140.24 47.38) (width 0.2) (layer "B.Cu") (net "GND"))
 (segment (start 142.78 47.38) (end 143.93 46.23) (width 0.2) (layer "B.Cu") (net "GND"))
 (segment (start 114.998301 52.301699) (end 118.53 48.77) (width 0.5) (layer "B.Cu") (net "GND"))
 (segment (start 97 52.301699) (end 114.998301 52.301699) (width 0.5) (layer "B.Cu") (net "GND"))
 (segment (start 122.38 45) (end 123.61 46.23) (width 0.2) (layer "B.Cu") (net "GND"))
 (segment (start 140.24 47.38) (end 142.78 47.38) (width 0.2) (layer "B.Cu") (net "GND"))
 (segment (start 130.08 45.08) (end 131.23 46.23) (width 0.2) (layer "B.Cu") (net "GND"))
 (segment (start 143.93 46.23) (end 145.08 45.08) (width 0.2) (layer "B.Cu") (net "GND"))
 (segment (start 114.68 45) (end 122.38 45) (width 0.2) (layer "B.Cu") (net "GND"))
 (segment (start 114.84 47.62) (end 117.38 47.62) (width 0.2) (layer "B.Cu") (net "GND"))
 (segment (start 156.63 48.77) (end 155.24 47.38) (width 0.2) (layer "B.Cu") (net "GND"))
 (segment (start 91.696769 49.301699) (end 88.696769 52.301699) (width 0.5) (layer "B.Cu") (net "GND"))
 (segment (start 150.16 47.38) (end 149.01 46.23) (width 0.2) (layer "B.Cu") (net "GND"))
 (segment (start 147.86 45.08) (end 149.01 46.23) (width 0.2) (layer "B.Cu") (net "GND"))
 (segment (start 132.38 45.08) (end 142.78 45.08) (width 0.2) (layer "B.Cu") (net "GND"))
 (segment (start 88.696769 52.301699) (end 88.696769 52.696769) (width 0.5) (layer "B.Cu") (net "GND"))
 (segment (start 131.23 46.23) (end 132.38 45.08) (width 0.2) (layer "B.Cu") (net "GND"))
 (segment (start 124.76 45.08) (end 130.08 45.08) (width 0.2) (layer "B.Cu") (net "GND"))
 (segment (start 110.91 54.09) (end 100 65) (width 0.2) (layer "F.Cu") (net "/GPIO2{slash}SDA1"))
 (segment (start 82.54 60.54) (end 82.54 47.5) (width 0.2) (layer "F.Cu") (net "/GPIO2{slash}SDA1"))
 (segment (start 100 65) (end 87 65) (width 0.2) (layer "F.Cu") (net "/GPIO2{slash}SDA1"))
 (segment (start 87 65) (end 82.54 60.54) (width 0.2) (layer "F.Cu") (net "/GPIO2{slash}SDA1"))
 (segment (start 110.91 48.77) (end 110.91 54.09) (width 0.2) (layer "F.Cu") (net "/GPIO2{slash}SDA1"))
 (segment (start 113.45 52.55) (end 113.45 48.77) (width 0.2) (layer "F.Cu") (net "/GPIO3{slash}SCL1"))
 (segment (start 100 66) (end 113.45 52.55) (width 0.2) (layer "F.Cu") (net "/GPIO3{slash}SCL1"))
 (segment (start 80 47.5) (end 80 60) (width 0.2) (layer "F.Cu") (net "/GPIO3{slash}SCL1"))
 (segment (start 86 66) (end 100 66) (width 0.2) (layer "F.Cu") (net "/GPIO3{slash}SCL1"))
 (segment (start 113.34 48.77) (end 113.45 48.77) (width 0.2) (layer "F.Cu") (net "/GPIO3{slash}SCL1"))
 (segment (start 80 60) (end 86 66) (width 0.2) (layer "F.Cu") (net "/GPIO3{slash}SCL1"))
 (segment (start 108.37 46.23) (end 110.91 46.23) (width 0.5) (layer "B.Cu") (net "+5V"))
 (segment (start 99 58) (end 99 61) (width 0.5) (layer "B.Cu") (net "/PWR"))
 (segment (start 96.301699 55.301699) (end 99 58) (width 0.5) (layer "B.Cu") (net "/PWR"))
 (segment (start 93.396769 55.301699) (end 96.301699 55.301699) (width 0.5) (layer "B.Cu") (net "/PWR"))
 (segment (start 93.396769 55.301699) (end 93.396769 55.603231) (width 0.2) (layer "B.Cu") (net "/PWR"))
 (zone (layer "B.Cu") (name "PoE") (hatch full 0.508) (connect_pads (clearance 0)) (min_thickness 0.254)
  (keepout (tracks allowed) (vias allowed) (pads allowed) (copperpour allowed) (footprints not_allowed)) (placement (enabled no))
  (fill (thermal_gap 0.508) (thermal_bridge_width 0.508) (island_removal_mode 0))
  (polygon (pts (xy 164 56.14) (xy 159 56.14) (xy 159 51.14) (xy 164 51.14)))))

